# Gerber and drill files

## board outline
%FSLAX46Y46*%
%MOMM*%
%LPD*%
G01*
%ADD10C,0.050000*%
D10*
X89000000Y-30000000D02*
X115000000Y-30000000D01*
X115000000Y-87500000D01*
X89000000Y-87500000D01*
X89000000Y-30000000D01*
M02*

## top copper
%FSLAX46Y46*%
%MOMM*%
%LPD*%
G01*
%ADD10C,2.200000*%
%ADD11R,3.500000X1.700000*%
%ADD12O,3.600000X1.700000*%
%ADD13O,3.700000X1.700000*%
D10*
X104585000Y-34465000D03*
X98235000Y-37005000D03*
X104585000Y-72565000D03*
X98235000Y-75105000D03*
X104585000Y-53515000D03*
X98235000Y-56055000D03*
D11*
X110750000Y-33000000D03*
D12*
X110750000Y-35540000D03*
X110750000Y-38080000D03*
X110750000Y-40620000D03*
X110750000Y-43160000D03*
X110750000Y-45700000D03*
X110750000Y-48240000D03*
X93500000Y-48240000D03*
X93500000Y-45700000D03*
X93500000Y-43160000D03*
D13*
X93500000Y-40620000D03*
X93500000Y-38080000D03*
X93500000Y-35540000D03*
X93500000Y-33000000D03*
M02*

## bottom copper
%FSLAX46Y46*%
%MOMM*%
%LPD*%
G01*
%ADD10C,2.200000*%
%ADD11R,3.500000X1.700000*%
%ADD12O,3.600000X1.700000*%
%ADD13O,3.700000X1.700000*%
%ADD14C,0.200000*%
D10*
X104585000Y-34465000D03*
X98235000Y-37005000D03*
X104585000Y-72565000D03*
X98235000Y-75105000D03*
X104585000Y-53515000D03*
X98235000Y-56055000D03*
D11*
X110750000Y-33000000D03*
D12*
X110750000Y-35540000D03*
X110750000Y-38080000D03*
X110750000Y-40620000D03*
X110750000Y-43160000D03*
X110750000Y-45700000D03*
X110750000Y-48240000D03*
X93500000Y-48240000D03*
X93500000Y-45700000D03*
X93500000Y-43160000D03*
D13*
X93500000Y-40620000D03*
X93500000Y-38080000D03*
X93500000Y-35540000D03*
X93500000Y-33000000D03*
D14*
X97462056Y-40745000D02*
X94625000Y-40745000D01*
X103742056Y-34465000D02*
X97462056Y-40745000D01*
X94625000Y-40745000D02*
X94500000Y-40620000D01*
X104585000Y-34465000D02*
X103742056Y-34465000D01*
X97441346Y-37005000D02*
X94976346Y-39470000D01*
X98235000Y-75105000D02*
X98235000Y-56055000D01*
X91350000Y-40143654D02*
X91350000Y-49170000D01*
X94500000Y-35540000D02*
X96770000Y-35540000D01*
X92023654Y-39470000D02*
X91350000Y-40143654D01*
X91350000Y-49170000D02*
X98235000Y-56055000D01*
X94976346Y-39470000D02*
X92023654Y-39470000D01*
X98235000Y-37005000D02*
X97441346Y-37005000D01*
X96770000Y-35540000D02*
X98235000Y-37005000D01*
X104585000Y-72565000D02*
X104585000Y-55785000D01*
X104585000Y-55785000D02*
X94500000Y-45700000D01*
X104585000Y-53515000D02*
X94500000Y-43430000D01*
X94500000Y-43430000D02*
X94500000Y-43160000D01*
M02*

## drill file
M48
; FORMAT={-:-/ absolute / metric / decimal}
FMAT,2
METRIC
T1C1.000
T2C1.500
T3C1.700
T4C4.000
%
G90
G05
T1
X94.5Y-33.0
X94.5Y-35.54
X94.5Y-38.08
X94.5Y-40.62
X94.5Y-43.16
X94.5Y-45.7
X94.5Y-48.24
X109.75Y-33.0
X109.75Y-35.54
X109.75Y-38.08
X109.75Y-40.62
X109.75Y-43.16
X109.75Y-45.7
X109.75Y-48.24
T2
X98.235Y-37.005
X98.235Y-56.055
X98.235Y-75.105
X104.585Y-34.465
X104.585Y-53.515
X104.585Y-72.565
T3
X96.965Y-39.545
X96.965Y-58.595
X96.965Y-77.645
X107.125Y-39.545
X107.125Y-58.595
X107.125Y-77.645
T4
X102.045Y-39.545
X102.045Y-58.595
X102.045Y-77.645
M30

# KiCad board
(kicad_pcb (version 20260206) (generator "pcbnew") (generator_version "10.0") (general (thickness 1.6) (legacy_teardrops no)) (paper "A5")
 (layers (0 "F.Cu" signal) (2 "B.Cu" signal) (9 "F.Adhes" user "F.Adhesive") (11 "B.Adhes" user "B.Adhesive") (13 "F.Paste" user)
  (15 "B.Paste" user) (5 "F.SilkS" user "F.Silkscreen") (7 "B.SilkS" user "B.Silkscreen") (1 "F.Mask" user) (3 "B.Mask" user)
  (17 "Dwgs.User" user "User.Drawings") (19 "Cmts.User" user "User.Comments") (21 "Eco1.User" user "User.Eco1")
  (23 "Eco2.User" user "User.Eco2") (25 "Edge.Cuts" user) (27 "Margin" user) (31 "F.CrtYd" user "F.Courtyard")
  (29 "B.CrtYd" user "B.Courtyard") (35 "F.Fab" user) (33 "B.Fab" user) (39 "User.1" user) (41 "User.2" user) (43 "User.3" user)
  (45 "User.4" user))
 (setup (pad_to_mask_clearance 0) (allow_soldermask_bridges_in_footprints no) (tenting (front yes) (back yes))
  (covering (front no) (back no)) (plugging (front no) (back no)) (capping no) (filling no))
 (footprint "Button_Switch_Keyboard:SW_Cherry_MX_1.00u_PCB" (layer "F.Cu") (at 104.585 34.465)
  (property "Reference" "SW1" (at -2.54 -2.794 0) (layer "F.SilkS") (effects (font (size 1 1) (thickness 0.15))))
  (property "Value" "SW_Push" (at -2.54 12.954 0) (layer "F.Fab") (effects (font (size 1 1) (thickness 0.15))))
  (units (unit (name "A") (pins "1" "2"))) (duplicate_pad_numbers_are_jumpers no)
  (pad "" np_thru_hole circle (at -7.62 5.08) (size 1.7 1.7) (drill 1.7) (layers "*.Cu" "*.Mask"))
  (pad "" np_thru_hole circle (at -2.54 5.08) (size 4 4) (drill 4) (layers "*.Cu" "*.Mask"))
  (pad "" np_thru_hole circle (at 2.54 5.08) (size 1.7 1.7) (drill 1.7) (layers "*.Cu" "*.Mask"))
  (pad "1" thru_hole circle (at 0 0) (size 2.2 2.2) (drill 1.5) (layers "*.Cu" "*.Mask") (remove_unused_layers no)
   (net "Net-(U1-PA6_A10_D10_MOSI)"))
  (pad "2" thru_hole circle (at -6.35 2.54) (size 2.2 2.2) (drill 1.5) (layers "*.Cu" "*.Mask") (remove_unused_layers no) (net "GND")))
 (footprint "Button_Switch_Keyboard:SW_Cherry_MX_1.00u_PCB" (layer "F.Cu") (at 104.585 72.565)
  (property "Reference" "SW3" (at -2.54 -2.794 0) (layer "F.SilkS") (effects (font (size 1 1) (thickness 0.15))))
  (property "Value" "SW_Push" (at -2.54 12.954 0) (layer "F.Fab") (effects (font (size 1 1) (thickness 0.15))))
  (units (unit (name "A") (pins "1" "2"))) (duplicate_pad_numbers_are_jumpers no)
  (pad "" np_thru_hole circle (at -7.62 5.08) (size 1.7 1.7) (drill 1.7) (layers "*.Cu" "*.Mask"))
  (pad "" np_thru_hole circle (at -2.54 5.08) (size 4 4) (drill 4) (layers "*.Cu" "*.Mask"))
  (pad "" np_thru_hole circle (at 2.54 5.08) (size 1.7 1.7) (drill 1.7) (layers "*.Cu" "*.Mask"))
  (pad "1" thru_hole circle (at 0 0) (size 2.2 2.2) (drill 1.5) (layers "*.Cu" "*.Mask") (remove_unused_layers no)
   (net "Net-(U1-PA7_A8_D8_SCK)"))
  (pad "2" thru_hole circle (at -6.35 2.54) (size 2.2 2.2) (drill 1.5) (layers "*.Cu" "*.Mask") (remove_unused_layers no) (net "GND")))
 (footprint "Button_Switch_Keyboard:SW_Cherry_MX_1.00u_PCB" (layer "F.Cu") (at 104.585 53.515)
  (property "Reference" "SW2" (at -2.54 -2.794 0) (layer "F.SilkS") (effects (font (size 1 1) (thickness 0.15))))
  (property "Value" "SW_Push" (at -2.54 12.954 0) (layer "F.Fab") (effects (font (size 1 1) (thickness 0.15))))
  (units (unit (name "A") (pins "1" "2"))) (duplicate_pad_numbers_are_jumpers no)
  (pad "" np_thru_hole circle (at -7.62 5.08) (size 1.7 1.7) (drill 1.7) (layers "*.Cu" "*.Mask"))
  (pad "" np_thru_hole circle (at -2.54 5.08) (size 4 4) (drill 4) (layers "*.Cu" "*.Mask"))
  (pad "" np_thru_hole circle (at 2.54 5.08) (size 1.7 1.7) (drill 1.7) (layers "*.Cu" "*.Mask"))
  (pad "1" thru_hole circle (at 0 0) (size 2.2 2.2) (drill 1.5) (layers "*.Cu" "*.Mask") (remove_unused_layers no)
   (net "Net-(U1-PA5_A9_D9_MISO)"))
  (pad "2" thru_hole circle (at -6.35 2.54) (size 2.2 2.2) (drill 1.5) (layers "*.Cu" "*.Mask") (remove_unused_layers no) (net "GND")))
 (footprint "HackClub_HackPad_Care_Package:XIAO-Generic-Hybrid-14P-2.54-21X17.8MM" (layer "B.Cu") (at 102.125 40.62 180)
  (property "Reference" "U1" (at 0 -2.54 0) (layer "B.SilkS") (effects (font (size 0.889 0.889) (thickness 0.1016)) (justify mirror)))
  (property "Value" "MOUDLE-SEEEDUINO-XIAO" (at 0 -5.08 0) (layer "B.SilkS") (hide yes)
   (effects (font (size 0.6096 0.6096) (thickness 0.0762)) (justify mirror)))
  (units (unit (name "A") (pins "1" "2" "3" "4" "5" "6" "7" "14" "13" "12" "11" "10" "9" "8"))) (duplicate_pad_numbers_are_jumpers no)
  (pad "1" thru_hole rect (at -7.625 7.62 180) (size 3.5 1.7) (drill 1 (offset -1 0)) (layers "*.Cu" "*.Mask") (remove_unused_layers no)
   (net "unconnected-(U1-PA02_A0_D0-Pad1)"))
  (pad "2" thru_hole oval (at -7.625 5.08 180) (size 3.6 1.7) (drill 1 (offset -1 0)) (layers "*.Cu" "*.Mask") (remove_unused_layers no)
   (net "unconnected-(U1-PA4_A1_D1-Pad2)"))
  (pad "3" thru_hole oval (at -7.625 2.54 180) (size 3.6 1.7) (drill 1 (offset -1 0)) (layers "*.Cu" "*.Mask") (remove_unused_layers no)
   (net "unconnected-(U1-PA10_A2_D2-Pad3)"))
  (pad "4" thru_hole oval (at -7.625 0 180) (size 3.6 1.7) (drill 1 (offset -1 0)) (layers "*.Cu" "*.Mask") (remove_unused_layers no)
   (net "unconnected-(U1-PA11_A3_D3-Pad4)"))
  (pad "5" thru_hole oval (at -7.625 -2.54 180) (size 3.6 1.7) (drill 1 (offset -1 0)) (layers "*.Cu" "*.Mask") (remove_unused_layers no)
   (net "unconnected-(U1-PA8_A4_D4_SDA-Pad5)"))
  (pad "6" thru_hole oval (at -7.625 -5.08) (size 3.6 1.7) (drill 1 (offset 1 0)) (layers "*.Cu" "*.Mask") (remove_unused_layers no)
   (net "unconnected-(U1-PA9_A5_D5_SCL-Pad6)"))
  (pad "7" thru_hole oval (at -7.625 -7.62 180) (size 3.6 1.7) (drill 1 (offset -1 0)) (layers "*.Cu" "*.Mask") (remove_unused_layers no)
   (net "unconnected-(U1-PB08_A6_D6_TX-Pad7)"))
  (pad "8" thru_hole oval (at 7.625 -7.62 180) (size 3.6 1.7) (drill 1 (offset 1 0)) (layers "*.Cu" "*.Mask") (remove_unused_layers no)
   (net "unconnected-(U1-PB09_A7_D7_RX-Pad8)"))
  (pad "9" thru_hole oval (at 7.625 -5.08 180) (size 3.6 1.7) (drill 1 (offset 1 0)) (layers "*.Cu" "*.Mask") (remove_unused_layers no)
   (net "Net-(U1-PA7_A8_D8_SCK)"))
  (pad "10" thru_hole oval (at 7.625 -2.54 180) (size 3.6 1.7) (drill 1 (offset 1 0)) (layers "*.Cu" "*.Mask") (remove_unused_layers no)
   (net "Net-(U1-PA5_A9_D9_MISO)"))
  (pad "11" thru_hole oval (at 7.625 0 180) (size 3.7 1.7) (drill 1 (offset 1 0)) (layers "*.Cu" "*.Mask") (remove_unused_layers no)
   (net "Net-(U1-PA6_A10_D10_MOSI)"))
  (pad "12" thru_hole oval (at 7.625 2.54 180) (size 3.7 1.7) (drill 1 (offset 1 0)) (layers "*.Cu" "*.Mask") (remove_unused_layers no)
   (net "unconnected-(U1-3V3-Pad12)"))
  (pad "13" thru_hole oval (at 7.625 5.08 180) (size 3.7 1.7) (drill 1 (offset 1 0)) (layers "*.Cu" "*.Mask") (remove_unused_layers no)
   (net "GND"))
  (pad "14" thru_hole oval (at 7.625 7.62 180) (size 3.7 1.7) (drill 1 (offset 1 0)) (layers "*.Cu" "*.Mask") (remove_unused_layers no)
   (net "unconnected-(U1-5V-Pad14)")))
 (gr_rect (start 89 30) (end 115 87.5) (stroke (width 0.05) (type default)) (fill no) (layer "Edge.Cuts"))
 (segment (start 97.462056 40.745) (end 94.625 40.745) (width 0.2) (layer "B.Cu") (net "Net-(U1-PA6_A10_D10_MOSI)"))
 (segment (start 103.742056 34.465) (end 97.462056 40.745) (width 0.2) (layer "B.Cu") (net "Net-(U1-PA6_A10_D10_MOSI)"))
 (segment (start 94.625 40.745) (end 94.5 40.62) (width 0.2) (layer "B.Cu") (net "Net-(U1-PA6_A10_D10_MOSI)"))
 (segment (start 104.585 34.465) (end 103.742056 34.465) (width 0.2) (layer "B.Cu") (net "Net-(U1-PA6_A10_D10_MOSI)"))
 (segment (start 97.441346 37.005) (end 94.976346 39.47) (width 0.2) (layer "B.Cu") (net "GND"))
 (segment (start 98.235 75.105) (end 98.235 56.055) (width 0.2) (layer "B.Cu") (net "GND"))
 (segment (start 91.35 40.143654) (end 91.35 49.17) (width 0.2) (layer "B.Cu") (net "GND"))
 (segment (start 94.5 35.54) (end 96.77 35.54) (width 0.2) (layer "B.Cu") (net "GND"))
 (segment (start 92.023654 39.47) (end 91.35 40.143654) (width 0.2) (layer "B.Cu") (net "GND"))
 (segment (start 91.35 49.17) (end 98.235 56.055) (width 0.2) (layer "B.Cu") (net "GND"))
 (segment (start 94.976346 39.47) (end 92.023654 39.47) (width 0.2) (layer "B.Cu") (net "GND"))
 (segment (start 98.235 37.005) (end 97.441346 37.005) (width 0.2) (layer "B.Cu") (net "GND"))
 (segment (start 96.77 35.54) (end 98.235 37.005) (width 0.2) (layer "B.Cu") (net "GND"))
 (segment (start 104.585 72.565) (end 104.585 55.785) (width 0.2) (layer "B.Cu") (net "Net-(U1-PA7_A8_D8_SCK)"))
 (segment (start 104.585 55.785) (end 94.5 45.7) (width 0.2) (layer "B.Cu") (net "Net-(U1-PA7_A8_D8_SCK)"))
 (segment (start 104.585 53.515) (end 94.5 43.43) (width 0.2) (layer "B.Cu") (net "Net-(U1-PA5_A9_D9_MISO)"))
 (segment (start 94.5 43.43) (end 94.5 43.16) (width 0.2) (layer "B.Cu") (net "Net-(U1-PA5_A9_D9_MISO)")))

